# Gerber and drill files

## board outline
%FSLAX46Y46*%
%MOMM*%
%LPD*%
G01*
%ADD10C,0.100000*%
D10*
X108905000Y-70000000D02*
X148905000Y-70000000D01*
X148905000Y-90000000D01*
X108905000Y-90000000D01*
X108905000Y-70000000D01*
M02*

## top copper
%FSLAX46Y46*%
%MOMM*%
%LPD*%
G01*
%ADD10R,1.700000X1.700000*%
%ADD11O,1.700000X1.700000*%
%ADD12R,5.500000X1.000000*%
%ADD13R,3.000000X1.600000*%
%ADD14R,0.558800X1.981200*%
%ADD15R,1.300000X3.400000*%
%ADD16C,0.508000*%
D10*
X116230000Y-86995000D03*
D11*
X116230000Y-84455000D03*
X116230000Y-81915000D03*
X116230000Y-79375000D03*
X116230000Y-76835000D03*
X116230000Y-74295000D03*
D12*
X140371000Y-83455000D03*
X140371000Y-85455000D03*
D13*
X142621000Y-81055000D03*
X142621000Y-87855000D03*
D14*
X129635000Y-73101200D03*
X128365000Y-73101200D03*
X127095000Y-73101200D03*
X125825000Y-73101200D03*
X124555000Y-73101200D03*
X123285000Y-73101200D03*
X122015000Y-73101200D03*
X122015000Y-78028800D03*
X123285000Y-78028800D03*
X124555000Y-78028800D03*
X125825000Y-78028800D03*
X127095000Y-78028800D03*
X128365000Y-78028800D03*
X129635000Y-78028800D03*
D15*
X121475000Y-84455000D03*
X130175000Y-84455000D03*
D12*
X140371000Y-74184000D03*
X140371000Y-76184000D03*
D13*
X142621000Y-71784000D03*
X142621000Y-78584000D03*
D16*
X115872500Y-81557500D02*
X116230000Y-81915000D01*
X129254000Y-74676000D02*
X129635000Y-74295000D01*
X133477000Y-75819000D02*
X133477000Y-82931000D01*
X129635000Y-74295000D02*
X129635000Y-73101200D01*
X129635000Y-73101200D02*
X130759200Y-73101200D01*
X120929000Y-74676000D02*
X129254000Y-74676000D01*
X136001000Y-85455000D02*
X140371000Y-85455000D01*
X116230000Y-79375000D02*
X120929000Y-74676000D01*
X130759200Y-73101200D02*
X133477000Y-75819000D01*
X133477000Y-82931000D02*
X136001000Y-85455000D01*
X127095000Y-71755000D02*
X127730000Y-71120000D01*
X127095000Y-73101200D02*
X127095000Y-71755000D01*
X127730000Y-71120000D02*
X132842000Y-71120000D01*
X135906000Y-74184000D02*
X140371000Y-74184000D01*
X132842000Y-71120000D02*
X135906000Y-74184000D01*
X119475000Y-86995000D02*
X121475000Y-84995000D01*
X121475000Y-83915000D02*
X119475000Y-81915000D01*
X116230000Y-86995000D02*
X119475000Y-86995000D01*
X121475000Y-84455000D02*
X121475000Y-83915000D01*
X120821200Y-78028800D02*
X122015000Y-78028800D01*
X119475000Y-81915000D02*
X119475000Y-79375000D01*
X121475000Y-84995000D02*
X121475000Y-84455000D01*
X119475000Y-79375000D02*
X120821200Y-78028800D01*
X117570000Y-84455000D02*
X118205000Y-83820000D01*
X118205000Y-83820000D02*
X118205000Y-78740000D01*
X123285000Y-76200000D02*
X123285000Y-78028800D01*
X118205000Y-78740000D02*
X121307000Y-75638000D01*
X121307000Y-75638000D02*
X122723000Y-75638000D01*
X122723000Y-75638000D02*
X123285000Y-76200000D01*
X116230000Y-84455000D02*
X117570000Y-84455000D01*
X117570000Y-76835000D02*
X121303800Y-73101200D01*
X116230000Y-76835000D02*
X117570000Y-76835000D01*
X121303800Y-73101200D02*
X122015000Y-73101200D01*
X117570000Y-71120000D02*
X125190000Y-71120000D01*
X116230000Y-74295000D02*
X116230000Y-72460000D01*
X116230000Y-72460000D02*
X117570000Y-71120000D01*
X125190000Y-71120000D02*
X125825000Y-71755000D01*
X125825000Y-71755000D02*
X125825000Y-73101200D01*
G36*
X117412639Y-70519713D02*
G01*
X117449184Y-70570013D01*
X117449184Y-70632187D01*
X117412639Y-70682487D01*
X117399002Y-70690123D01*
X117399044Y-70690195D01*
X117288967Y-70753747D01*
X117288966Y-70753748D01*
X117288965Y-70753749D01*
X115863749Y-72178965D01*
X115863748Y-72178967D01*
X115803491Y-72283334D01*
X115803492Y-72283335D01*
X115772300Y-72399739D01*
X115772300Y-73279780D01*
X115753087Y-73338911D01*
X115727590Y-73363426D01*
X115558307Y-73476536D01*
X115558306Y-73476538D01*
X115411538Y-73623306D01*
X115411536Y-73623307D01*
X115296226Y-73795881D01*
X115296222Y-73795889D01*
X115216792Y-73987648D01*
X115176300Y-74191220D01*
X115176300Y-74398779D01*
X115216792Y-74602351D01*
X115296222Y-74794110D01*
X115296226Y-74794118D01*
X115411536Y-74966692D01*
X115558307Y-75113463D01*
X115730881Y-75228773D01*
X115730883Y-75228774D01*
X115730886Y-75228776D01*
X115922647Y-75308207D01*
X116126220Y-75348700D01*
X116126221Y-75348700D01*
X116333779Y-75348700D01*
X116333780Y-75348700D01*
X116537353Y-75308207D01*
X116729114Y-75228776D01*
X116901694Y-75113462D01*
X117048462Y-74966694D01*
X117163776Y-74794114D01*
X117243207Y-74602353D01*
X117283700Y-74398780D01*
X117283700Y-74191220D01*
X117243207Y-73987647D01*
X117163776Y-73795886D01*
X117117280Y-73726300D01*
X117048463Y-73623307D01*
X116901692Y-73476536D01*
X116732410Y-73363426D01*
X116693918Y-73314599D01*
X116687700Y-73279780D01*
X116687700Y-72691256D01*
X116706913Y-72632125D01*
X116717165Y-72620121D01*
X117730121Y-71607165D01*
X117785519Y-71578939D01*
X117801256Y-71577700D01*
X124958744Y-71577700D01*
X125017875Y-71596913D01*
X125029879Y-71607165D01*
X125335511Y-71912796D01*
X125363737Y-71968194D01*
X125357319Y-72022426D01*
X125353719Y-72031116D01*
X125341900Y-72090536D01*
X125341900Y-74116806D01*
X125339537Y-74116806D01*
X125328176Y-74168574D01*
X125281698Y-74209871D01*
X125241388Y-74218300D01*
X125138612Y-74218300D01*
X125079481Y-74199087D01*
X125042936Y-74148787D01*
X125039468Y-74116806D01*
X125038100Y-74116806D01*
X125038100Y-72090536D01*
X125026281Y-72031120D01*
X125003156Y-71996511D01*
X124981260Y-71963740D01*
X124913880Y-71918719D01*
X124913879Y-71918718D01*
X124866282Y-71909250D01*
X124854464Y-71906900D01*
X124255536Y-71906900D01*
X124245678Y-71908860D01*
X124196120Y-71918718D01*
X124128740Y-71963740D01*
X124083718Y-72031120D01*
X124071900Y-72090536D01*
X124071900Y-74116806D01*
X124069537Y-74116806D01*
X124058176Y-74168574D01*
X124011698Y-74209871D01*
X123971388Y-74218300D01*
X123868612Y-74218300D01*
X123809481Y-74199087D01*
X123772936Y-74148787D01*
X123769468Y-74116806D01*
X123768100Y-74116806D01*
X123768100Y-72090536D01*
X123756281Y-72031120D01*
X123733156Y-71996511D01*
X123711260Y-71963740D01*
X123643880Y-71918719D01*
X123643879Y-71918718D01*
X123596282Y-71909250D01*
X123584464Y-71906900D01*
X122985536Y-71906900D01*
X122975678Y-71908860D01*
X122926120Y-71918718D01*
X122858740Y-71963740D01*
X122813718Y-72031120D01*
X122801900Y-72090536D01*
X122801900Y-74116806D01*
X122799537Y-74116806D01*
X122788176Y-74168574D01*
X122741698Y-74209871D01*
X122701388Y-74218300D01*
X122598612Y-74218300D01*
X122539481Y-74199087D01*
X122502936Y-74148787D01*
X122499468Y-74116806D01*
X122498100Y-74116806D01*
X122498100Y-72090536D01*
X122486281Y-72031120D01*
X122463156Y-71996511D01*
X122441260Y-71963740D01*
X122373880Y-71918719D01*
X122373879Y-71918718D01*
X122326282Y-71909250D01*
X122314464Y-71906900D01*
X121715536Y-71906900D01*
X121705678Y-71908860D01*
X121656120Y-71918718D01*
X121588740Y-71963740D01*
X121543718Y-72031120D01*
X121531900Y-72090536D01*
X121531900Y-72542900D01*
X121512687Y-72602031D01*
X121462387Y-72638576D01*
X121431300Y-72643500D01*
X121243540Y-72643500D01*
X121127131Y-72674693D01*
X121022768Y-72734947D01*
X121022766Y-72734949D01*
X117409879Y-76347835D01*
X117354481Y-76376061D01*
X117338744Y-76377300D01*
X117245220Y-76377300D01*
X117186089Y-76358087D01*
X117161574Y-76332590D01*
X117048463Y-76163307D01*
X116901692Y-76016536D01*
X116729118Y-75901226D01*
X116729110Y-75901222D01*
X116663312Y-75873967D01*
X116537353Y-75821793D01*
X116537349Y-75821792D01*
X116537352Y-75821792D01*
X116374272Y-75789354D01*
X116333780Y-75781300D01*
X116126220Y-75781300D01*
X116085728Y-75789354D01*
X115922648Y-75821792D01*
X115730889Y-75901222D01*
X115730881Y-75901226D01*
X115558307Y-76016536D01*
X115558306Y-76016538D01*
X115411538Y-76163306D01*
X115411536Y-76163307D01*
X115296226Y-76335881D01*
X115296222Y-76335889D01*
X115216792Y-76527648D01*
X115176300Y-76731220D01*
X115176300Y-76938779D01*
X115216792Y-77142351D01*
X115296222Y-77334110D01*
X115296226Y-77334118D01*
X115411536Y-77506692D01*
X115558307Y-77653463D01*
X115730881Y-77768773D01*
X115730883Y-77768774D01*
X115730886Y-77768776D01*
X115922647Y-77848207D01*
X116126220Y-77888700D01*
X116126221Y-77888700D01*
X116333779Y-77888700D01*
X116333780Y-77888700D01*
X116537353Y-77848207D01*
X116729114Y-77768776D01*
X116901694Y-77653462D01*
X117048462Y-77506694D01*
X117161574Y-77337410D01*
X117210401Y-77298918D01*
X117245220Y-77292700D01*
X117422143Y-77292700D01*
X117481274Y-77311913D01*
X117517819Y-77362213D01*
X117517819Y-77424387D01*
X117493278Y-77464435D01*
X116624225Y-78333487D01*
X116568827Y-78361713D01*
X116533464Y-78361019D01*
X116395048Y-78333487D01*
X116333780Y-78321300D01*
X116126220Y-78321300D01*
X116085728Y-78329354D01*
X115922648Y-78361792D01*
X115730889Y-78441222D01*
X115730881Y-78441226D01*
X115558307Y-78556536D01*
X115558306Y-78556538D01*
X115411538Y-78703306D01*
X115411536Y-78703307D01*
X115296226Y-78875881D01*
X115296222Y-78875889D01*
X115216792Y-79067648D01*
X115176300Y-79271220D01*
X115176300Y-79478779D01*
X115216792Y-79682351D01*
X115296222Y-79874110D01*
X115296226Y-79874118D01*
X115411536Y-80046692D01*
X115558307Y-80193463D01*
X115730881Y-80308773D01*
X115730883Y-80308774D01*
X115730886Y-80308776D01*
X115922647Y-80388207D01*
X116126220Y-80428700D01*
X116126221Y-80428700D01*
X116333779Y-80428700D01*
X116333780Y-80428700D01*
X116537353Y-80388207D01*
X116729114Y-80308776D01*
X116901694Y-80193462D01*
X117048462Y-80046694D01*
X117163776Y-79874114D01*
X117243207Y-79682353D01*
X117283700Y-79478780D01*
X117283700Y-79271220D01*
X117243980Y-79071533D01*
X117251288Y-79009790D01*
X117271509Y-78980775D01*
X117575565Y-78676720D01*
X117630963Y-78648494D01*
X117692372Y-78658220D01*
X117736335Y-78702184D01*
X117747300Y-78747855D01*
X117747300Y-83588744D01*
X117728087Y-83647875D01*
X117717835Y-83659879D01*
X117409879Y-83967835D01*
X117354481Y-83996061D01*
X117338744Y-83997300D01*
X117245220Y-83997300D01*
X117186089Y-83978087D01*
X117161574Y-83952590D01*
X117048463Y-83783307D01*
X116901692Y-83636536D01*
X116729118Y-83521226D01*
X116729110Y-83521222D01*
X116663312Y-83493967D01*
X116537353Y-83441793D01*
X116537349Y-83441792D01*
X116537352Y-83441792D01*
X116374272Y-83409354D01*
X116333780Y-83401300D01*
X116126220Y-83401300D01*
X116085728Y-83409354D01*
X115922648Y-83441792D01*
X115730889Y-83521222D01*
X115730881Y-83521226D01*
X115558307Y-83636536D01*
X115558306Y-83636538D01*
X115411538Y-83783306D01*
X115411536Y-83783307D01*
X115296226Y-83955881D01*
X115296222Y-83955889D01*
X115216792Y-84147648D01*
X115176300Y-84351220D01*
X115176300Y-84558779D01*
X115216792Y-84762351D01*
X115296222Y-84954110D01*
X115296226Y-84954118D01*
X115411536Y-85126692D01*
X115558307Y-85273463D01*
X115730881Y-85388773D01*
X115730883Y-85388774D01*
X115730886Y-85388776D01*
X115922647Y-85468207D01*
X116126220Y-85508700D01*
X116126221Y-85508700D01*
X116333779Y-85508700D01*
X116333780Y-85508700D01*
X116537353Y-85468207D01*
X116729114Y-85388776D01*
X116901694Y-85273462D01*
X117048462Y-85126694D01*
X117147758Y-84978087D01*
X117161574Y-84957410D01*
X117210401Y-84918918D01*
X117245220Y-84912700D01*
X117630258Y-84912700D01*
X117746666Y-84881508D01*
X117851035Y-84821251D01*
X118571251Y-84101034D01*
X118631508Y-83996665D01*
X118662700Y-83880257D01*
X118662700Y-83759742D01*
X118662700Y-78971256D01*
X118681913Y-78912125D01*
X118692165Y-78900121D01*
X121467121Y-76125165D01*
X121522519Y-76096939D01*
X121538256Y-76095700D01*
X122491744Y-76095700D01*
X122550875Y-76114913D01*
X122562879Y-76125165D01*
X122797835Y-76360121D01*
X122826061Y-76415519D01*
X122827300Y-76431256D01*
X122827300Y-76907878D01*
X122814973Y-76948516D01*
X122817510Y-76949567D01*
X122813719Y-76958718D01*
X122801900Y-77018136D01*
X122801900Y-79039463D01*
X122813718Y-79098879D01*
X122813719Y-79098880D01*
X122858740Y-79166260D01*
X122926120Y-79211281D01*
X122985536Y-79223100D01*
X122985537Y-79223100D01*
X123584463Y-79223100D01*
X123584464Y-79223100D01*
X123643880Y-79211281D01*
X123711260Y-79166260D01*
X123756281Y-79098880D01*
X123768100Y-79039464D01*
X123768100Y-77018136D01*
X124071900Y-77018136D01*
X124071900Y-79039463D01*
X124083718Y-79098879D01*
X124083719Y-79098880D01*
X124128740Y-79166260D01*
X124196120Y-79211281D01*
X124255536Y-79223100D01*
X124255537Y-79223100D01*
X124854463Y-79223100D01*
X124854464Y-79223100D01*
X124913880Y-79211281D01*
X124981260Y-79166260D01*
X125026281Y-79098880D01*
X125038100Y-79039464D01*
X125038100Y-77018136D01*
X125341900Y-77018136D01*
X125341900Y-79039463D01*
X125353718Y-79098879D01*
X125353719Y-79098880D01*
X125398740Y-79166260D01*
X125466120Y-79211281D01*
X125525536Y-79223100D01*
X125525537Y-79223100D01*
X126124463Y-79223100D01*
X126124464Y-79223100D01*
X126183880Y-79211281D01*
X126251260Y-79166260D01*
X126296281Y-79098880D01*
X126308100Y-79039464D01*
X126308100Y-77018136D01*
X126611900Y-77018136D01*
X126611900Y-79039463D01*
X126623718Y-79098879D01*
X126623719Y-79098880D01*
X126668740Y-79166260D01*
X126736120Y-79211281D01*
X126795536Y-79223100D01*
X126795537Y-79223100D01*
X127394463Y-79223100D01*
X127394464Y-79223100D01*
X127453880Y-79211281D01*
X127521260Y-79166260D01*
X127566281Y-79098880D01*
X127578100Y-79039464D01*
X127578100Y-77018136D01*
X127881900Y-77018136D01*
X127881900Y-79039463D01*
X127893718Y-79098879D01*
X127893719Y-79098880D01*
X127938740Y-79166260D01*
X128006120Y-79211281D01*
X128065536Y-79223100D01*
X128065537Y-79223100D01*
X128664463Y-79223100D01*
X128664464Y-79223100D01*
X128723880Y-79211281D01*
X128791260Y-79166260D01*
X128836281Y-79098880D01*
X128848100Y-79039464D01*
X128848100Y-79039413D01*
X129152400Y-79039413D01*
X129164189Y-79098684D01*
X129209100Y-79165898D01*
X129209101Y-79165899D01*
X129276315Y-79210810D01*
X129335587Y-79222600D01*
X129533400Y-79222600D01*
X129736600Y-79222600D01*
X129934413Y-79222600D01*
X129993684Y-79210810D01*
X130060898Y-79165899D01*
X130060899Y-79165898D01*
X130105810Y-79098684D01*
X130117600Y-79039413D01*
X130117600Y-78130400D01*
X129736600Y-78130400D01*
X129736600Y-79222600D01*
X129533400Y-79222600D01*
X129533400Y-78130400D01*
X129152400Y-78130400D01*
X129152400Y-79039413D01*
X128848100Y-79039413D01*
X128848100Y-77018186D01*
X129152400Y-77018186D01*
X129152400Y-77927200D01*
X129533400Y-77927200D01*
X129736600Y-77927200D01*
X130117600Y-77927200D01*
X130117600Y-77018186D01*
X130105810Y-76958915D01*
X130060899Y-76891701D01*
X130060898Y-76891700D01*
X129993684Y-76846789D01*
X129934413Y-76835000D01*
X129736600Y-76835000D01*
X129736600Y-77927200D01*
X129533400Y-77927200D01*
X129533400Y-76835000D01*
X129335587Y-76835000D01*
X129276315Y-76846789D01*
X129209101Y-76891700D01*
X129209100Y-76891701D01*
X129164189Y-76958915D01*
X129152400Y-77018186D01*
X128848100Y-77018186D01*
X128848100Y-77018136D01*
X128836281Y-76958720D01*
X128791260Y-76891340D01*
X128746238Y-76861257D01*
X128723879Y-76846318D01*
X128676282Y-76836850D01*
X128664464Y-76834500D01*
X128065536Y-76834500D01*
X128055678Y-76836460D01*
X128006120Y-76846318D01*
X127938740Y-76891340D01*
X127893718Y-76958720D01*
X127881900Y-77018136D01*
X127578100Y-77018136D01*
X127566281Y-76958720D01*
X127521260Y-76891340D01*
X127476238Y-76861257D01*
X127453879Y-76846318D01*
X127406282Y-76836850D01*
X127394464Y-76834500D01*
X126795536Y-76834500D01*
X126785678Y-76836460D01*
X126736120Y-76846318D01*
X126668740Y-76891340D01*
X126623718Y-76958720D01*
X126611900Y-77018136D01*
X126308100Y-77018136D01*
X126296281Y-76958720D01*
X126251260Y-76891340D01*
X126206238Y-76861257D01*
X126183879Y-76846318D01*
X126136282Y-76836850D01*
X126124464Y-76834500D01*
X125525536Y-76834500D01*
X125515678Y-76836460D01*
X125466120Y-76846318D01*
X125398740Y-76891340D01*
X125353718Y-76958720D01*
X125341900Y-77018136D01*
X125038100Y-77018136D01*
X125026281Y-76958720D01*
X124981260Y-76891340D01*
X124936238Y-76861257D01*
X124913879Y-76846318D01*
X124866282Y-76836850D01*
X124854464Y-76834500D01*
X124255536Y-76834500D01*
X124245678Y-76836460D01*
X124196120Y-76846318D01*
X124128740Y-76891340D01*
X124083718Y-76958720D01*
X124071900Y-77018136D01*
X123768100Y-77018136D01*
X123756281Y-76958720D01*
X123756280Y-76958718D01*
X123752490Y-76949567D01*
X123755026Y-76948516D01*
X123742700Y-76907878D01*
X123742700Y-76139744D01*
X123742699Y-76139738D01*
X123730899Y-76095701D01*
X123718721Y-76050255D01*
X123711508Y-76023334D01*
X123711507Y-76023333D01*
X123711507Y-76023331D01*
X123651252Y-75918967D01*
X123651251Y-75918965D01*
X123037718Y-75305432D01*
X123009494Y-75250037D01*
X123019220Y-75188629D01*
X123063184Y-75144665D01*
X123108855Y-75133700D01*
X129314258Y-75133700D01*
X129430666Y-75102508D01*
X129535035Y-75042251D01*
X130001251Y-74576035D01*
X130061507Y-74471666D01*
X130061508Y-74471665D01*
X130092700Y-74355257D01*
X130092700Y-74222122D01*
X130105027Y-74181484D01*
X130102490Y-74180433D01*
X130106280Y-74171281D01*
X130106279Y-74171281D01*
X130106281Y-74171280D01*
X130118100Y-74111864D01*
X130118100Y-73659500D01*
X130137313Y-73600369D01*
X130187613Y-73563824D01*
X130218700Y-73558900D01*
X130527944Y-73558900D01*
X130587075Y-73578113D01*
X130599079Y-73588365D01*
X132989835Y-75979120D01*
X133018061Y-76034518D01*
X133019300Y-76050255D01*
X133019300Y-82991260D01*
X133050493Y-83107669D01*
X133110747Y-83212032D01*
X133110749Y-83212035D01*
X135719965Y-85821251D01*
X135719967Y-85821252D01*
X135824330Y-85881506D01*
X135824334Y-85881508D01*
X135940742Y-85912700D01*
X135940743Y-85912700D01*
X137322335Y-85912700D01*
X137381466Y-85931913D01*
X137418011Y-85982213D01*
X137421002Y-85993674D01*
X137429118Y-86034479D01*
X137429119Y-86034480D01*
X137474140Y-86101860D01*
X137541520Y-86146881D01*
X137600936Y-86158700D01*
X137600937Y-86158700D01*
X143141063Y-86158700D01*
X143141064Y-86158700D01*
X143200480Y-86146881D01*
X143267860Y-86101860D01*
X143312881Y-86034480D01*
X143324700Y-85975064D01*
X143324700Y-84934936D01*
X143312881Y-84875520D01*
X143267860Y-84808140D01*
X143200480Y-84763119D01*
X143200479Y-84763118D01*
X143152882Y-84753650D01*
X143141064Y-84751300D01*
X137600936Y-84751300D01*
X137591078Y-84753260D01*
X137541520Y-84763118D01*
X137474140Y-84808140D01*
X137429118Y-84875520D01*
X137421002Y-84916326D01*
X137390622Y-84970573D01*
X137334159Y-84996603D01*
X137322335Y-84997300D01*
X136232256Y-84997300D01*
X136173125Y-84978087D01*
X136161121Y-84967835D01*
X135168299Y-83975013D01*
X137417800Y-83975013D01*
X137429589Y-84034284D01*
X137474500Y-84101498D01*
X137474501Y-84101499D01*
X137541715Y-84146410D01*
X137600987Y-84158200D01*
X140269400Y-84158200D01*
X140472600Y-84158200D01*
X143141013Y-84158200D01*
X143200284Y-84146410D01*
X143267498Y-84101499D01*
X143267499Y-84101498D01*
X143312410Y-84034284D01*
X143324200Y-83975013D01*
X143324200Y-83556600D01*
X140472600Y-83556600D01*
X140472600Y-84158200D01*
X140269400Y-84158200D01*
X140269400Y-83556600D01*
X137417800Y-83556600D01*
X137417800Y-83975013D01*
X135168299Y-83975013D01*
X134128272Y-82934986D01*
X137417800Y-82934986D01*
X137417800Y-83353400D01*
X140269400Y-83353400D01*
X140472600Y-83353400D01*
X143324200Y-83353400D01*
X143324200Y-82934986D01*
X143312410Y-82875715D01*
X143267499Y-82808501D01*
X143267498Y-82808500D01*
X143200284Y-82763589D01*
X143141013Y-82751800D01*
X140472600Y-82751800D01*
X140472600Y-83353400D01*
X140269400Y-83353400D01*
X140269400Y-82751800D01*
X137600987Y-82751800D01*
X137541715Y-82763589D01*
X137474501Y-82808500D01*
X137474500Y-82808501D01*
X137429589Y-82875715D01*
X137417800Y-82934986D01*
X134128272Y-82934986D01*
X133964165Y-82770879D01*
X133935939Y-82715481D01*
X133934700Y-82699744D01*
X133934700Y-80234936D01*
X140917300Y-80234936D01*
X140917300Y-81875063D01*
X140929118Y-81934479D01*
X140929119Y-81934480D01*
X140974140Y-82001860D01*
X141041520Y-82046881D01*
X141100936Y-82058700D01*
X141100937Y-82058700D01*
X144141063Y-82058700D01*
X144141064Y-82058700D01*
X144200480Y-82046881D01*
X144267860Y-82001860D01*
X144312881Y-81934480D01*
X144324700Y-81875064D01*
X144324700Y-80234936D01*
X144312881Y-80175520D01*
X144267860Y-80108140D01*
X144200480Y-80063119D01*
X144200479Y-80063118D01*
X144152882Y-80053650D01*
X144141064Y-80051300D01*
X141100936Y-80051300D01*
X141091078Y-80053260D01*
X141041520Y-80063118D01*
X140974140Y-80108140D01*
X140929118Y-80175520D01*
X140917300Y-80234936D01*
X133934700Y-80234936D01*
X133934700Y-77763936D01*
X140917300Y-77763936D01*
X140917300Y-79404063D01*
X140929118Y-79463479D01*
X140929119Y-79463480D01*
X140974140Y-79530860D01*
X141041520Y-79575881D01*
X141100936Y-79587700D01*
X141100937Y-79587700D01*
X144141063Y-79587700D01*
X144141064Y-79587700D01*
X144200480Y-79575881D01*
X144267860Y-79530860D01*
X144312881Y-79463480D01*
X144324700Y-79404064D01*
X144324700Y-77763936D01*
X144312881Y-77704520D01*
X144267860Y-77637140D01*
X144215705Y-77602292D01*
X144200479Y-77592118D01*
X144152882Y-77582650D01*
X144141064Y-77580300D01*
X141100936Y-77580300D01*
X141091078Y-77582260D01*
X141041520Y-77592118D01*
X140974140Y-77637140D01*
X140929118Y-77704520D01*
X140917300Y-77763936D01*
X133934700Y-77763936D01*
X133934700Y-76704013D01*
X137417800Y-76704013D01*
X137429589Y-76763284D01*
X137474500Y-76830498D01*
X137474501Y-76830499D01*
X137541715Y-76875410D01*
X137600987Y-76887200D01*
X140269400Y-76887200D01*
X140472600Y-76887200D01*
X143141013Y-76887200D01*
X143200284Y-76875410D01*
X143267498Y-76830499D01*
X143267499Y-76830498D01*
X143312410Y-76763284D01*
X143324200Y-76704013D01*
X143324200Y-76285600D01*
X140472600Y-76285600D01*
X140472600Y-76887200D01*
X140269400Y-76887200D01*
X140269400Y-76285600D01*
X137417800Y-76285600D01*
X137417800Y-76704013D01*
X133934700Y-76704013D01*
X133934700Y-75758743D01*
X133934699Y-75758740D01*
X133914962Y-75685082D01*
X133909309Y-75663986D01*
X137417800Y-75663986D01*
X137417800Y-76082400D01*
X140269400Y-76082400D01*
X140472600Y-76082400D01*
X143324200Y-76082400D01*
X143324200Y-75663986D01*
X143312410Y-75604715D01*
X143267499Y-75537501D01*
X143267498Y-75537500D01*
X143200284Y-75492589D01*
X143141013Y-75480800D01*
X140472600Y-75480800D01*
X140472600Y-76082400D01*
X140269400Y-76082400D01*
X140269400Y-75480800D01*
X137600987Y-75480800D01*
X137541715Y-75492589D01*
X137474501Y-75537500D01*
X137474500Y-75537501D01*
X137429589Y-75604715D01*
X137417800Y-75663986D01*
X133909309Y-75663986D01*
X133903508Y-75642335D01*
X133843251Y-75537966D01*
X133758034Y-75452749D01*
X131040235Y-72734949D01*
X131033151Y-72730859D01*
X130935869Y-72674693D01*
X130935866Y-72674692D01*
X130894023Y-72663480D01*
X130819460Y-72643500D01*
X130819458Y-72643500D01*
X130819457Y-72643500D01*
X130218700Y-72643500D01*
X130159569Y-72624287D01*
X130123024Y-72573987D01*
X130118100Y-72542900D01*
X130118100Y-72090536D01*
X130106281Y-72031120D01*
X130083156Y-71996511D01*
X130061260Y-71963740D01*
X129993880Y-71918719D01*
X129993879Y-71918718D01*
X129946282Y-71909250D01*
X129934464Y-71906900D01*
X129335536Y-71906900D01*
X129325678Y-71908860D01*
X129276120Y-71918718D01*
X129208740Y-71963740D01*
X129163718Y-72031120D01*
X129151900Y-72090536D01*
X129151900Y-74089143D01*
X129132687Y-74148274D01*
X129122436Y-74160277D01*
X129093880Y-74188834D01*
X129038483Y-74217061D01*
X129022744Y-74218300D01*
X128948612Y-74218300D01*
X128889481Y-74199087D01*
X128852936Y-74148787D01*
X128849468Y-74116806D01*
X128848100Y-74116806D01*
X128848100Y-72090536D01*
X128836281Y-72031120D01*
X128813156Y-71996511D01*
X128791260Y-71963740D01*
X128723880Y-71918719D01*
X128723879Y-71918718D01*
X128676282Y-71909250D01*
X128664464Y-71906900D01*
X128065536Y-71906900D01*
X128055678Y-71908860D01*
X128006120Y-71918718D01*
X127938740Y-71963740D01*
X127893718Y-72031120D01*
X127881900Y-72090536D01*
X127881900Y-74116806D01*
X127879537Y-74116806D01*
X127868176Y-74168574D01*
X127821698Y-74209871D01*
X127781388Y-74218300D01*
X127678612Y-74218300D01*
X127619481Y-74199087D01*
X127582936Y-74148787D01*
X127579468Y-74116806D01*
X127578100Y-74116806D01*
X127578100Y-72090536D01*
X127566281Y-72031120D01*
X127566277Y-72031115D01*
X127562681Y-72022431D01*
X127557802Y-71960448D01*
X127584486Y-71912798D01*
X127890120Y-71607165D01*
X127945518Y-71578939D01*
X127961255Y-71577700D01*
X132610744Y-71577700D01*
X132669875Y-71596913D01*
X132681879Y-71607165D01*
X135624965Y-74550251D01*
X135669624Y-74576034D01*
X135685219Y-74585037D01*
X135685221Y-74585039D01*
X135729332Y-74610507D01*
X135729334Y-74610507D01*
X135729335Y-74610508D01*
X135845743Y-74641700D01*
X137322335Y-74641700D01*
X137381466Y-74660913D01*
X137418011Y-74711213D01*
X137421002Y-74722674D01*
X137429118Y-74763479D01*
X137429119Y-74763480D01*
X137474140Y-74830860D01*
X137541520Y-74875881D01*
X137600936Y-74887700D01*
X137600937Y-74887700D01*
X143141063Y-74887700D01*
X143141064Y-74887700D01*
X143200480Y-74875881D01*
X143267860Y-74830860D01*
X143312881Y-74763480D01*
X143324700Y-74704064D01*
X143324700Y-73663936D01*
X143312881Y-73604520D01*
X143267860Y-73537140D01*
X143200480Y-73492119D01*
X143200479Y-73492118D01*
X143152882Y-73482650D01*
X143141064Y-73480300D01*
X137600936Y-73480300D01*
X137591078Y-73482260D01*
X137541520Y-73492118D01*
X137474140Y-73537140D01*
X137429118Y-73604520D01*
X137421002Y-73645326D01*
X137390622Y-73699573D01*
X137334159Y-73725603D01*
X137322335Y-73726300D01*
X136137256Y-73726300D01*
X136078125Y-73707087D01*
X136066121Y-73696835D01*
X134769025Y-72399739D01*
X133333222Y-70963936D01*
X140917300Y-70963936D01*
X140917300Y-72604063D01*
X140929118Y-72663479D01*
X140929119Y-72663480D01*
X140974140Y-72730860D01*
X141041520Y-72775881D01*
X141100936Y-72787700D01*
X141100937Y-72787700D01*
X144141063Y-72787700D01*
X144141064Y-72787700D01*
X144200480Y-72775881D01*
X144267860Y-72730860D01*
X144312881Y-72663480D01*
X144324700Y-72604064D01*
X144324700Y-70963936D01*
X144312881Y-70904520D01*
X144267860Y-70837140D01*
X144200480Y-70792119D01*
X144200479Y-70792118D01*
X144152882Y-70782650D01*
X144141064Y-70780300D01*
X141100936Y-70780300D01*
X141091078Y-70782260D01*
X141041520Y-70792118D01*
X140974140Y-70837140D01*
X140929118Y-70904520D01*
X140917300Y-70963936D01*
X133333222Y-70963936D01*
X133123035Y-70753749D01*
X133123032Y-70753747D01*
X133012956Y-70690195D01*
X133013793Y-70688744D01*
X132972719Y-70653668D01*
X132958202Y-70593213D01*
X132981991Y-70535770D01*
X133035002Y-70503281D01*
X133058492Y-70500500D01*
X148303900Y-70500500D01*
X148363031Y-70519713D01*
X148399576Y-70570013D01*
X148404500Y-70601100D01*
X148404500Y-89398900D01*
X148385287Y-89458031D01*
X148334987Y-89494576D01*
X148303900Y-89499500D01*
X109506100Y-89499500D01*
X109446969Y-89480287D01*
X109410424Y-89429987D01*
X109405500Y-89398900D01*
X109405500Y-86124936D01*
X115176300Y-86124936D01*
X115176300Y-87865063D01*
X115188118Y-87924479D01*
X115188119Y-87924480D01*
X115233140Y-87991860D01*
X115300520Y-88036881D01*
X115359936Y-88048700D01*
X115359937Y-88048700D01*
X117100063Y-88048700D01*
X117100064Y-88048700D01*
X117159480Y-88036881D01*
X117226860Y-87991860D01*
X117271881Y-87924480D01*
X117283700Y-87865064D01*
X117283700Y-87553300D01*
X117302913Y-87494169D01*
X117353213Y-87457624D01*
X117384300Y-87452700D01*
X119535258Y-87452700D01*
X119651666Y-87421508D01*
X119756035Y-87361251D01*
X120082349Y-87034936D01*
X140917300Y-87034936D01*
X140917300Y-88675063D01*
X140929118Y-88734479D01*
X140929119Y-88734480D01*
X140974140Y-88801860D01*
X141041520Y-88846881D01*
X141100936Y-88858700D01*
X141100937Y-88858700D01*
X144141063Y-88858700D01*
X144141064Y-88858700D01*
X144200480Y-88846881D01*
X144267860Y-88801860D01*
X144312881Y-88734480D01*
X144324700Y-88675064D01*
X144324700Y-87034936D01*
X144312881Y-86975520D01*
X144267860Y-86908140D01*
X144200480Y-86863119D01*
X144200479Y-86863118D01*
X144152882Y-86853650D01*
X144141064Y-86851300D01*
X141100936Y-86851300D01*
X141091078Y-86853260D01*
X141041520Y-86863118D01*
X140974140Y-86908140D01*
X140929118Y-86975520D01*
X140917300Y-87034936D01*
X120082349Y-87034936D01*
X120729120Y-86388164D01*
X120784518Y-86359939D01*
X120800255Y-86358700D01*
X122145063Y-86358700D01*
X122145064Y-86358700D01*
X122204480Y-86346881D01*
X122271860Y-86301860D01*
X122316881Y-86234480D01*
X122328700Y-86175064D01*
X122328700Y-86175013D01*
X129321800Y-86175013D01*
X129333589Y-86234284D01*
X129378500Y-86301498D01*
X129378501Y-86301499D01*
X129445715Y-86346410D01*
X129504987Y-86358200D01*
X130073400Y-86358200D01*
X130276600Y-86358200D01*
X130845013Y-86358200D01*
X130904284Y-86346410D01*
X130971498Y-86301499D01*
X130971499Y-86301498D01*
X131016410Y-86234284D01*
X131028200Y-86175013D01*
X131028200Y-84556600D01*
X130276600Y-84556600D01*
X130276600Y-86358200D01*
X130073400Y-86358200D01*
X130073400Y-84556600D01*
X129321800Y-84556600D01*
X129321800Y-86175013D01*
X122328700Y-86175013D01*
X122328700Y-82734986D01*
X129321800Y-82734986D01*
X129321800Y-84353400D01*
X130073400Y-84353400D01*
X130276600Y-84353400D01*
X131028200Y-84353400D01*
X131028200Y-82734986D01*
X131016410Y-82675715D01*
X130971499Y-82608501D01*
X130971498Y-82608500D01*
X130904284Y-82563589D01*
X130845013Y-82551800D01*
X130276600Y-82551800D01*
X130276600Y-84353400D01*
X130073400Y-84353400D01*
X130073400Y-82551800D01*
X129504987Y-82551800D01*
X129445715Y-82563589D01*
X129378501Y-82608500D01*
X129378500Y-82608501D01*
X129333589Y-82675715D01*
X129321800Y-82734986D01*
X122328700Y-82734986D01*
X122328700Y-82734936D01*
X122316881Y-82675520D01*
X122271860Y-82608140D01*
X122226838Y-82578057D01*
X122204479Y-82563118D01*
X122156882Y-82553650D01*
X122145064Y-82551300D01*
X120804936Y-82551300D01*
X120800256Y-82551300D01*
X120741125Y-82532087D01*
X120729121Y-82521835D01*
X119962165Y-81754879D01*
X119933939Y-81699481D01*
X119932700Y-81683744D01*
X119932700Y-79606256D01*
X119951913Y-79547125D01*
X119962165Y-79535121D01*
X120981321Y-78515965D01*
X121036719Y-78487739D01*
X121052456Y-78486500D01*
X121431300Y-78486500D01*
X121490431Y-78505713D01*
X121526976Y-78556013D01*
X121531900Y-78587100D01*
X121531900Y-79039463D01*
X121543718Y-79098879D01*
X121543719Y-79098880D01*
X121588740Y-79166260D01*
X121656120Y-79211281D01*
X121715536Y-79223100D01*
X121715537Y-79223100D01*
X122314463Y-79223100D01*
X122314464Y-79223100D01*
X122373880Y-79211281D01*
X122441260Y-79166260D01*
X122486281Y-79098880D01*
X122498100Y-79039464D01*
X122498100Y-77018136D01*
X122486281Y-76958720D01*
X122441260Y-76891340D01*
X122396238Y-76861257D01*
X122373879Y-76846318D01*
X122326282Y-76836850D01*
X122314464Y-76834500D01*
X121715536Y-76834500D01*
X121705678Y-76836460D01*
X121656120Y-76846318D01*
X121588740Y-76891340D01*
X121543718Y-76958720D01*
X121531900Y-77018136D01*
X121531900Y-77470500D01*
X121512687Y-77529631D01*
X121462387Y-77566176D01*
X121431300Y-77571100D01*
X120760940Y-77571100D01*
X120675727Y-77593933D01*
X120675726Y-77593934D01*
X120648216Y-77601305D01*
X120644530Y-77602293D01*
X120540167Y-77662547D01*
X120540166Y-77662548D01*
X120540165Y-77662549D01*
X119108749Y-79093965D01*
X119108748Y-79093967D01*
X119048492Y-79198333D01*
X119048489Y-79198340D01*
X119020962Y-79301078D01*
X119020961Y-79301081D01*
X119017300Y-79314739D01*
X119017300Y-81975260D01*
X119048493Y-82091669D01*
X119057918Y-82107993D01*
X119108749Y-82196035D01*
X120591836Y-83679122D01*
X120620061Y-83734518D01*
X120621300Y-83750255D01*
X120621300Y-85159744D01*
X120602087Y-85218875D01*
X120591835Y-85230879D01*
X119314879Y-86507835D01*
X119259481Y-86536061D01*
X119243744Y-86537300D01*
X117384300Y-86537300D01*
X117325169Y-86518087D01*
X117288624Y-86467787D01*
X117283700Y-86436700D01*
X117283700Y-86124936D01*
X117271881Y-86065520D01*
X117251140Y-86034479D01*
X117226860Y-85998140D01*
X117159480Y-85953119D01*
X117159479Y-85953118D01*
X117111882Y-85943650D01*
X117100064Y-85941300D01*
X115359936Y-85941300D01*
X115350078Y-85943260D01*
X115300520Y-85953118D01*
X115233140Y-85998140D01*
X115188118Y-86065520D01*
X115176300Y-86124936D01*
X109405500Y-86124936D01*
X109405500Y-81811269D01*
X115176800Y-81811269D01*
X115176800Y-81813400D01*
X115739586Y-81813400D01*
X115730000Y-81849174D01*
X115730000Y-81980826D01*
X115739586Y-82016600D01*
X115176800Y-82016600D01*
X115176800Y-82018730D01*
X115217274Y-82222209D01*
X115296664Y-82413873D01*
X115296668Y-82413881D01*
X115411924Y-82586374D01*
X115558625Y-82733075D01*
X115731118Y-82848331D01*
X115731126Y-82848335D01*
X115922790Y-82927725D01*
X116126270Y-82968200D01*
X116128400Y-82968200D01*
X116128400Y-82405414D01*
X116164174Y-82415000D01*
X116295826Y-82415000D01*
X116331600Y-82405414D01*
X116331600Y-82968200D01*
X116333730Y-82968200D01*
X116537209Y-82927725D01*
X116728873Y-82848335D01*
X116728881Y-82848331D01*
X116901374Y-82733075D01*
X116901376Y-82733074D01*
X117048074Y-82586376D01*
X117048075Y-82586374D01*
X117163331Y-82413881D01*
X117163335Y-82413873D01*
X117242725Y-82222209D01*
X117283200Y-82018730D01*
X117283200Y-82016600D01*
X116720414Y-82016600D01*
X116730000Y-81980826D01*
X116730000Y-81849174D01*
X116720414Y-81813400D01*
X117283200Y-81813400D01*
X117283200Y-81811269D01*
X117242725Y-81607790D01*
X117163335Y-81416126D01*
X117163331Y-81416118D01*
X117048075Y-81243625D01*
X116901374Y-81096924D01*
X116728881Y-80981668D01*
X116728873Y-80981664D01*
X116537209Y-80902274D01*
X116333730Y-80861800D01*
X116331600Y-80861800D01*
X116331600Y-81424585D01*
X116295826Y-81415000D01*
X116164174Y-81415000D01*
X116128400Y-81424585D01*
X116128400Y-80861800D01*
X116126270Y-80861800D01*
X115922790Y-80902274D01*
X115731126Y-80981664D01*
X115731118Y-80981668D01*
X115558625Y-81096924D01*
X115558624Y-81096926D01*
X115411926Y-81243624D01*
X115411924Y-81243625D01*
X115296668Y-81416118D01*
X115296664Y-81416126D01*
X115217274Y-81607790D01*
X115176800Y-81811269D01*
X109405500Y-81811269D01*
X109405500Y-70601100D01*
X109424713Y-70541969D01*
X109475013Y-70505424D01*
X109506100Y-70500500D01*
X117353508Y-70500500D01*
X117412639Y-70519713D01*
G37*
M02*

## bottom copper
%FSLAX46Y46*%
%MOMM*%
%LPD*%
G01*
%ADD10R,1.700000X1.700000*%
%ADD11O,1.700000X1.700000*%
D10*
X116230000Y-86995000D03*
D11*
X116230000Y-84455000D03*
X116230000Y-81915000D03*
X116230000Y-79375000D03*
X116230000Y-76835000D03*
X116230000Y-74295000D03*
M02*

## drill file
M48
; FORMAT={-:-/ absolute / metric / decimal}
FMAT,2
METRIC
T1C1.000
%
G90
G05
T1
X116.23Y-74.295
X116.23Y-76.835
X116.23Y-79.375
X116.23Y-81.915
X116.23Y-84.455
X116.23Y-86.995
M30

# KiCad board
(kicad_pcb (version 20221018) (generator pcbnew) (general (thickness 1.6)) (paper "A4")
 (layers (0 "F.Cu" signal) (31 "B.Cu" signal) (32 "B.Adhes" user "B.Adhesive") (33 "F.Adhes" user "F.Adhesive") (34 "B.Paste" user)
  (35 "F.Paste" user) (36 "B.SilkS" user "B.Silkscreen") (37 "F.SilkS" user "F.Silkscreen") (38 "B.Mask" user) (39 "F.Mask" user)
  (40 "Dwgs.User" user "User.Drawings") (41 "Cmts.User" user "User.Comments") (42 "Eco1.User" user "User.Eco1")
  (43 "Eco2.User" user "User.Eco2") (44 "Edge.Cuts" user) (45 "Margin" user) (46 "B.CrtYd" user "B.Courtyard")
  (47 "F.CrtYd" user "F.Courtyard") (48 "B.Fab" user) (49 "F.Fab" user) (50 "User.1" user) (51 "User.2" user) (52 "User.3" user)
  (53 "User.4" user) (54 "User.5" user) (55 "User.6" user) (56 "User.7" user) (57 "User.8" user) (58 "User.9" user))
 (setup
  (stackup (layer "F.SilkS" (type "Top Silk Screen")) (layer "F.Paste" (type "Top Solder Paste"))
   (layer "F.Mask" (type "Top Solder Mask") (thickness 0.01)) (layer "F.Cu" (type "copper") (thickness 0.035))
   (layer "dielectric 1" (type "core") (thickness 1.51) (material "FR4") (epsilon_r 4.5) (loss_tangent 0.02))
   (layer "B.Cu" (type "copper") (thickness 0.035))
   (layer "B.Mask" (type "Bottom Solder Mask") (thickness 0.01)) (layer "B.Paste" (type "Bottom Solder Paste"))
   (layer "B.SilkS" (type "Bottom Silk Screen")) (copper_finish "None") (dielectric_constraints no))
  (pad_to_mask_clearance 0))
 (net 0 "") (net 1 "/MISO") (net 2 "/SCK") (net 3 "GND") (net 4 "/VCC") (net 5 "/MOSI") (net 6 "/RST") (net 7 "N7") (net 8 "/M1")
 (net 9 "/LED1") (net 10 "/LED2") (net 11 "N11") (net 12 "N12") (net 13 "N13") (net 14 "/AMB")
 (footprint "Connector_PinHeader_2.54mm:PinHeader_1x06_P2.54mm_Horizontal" (layer "F.Cu") (at 116.23 86.995 180)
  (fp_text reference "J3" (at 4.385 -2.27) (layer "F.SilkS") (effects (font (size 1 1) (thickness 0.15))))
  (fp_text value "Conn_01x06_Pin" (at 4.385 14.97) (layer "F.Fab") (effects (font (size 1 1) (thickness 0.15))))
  (pad "1" thru_hole rect (at 0 0 180) (size 1.7 1.7) (drill 1) (layers "*.Cu" "*.Mask") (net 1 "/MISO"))
  (pad "2" thru_hole oval (at 0 2.54 180) (size 1.7 1.7) (drill 1) (layers "*.Cu" "*.Mask") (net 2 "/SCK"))
  (pad "3" thru_hole oval (at 0 5.08 180) (size 1.7 1.7) (drill 1) (layers "*.Cu" "*.Mask") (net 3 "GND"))
  (pad "4" thru_hole oval (at 0 7.62 180) (size 1.7 1.7) (drill 1) (layers "*.Cu" "*.Mask") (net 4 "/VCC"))
  (pad "5" thru_hole oval (at 0 10.16 180) (size 1.7 1.7) (drill 1) (layers "*.Cu" "*.Mask") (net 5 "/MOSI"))
  (pad "6" thru_hole oval (at 0 12.7 180) (size 1.7 1.7) (drill 1) (layers "*.Cu" "*.Mask") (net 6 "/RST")))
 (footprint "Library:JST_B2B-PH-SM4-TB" (layer "F.Cu") (at 142.621 84.455 -90)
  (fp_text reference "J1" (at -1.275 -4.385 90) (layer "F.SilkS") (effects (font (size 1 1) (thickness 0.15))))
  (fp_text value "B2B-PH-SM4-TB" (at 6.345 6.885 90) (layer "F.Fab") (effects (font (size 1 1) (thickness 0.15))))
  (pad "1" smd rect (at -1 2.25 270) (size 1 5.5) (layers "F.Cu" "F.Paste" "F.Mask") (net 3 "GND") (solder_mask_margin 0.102))
  (pad "2" smd rect (at 1 2.25 270) (size 1 5.5) (layers "F.Cu" "F.Paste" "F.Mask") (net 4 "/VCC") (solder_mask_margin 0.102))
  (pad "S1" smd rect (at -3.4 0 270) (size 1.6 3) (layers "F.Cu" "F.Paste" "F.Mask") (solder_mask_margin 0.102))
  (pad "S2" smd rect (at 3.4 0 270) (size 1.6 3) (layers "F.Cu" "F.Paste" "F.Mask") (solder_mask_margin 0.102)))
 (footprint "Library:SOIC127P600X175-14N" (layer "F.Cu") (at 125.825 75.565 -90)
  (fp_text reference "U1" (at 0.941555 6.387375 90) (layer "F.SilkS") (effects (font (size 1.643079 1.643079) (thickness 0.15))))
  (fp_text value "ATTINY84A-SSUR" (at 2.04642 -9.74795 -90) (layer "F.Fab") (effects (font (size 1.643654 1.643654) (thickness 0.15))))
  (pad "1" smd rect (at -2.4638 -3.81 270) (size 1.9812 0.5588) (layers "F.Cu" "F.Paste" "F.Mask") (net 4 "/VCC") (solder_mask_margin 0.102))
  (pad "2" smd rect (at -2.4638 -2.54 270) (size 1.9812 0.5588) (layers "F.Cu" "F.Paste" "F.Mask") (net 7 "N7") (solder_mask_margin 0.102))
  (pad "3" smd rect (at -2.4638 -1.27 270) (size 1.9812 0.5588) (layers "F.Cu" "F.Paste" "F.Mask") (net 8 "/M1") (solder_mask_margin 0.102))
  (pad "4" smd rect (at -2.4638 0 270) (size 1.9812 0.5588) (layers "F.Cu" "F.Paste" "F.Mask") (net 6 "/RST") (solder_mask_margin 0.102))
  (pad "5" smd rect (at -2.4638 1.27 270) (size 1.9812 0.5588) (layers "F.Cu" "F.Paste" "F.Mask") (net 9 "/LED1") (solder_mask_margin 0.102))
  (pad "6" smd rect (at -2.4638 2.54 270) (size 1.9812 0.5588) (layers "F.Cu" "F.Paste" "F.Mask") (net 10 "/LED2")
   (solder_mask_margin 0.102))
  (pad "7" smd rect (at -2.4638 3.81 270) (size 1.9812 0.5588) (layers "F.Cu" "F.Paste" "F.Mask") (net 5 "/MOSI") (solder_mask_margin 0.102))
  (pad "8" smd rect (at 2.4638 3.81 270) (size 1.9812 0.5588) (layers "F.Cu" "F.Paste" "F.Mask") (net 1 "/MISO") (solder_mask_margin 0.102))
  (pad "9" smd rect (at 2.4638 2.54 270) (size 1.9812 0.5588) (layers "F.Cu" "F.Paste" "F.Mask") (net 2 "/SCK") (solder_mask_margin 0.102))
  (pad "10" smd rect (at 2.4638 1.27 270) (size 1.9812 0.5588) (layers "F.Cu" "F.Paste" "F.Mask") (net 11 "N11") (solder_mask_margin 0.102))
  (pad "11" smd rect (at 2.4638 0 270) (size 1.9812 0.5588) (layers "F.Cu" "F.Paste" "F.Mask") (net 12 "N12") (solder_mask_margin 0.102))
  (pad "12" smd rect (at 2.4638 -1.27 270) (size 1.9812 0.5588) (layers "F.Cu" "F.Paste" "F.Mask") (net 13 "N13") (solder_mask_margin 0.102))
  (pad "13" smd rect (at 2.4638 -2.54 270) (size 1.9812 0.5588) (layers "F.Cu" "F.Paste" "F.Mask") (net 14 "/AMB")
   (solder_mask_margin 0.102))
  (pad "14" smd rect (at 2.4638 -3.81 270) (size 1.9812 0.5588) (layers "F.Cu" "F.Paste" "F.Mask") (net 3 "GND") (solder_mask_margin 0.102)))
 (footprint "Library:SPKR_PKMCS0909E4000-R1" (layer "F.Cu") (at 125.825 84.455)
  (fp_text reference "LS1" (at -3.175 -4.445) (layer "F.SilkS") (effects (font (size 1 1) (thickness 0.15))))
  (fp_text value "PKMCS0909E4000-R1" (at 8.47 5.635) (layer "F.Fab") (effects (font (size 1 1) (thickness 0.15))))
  (pad "1" smd rect (at -4.35 0) (size 1.3 3.4) (layers "F.Cu" "F.Paste" "F.Mask") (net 1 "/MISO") (solder_mask_margin 0.102))
  (pad "2" smd rect (at 4.35 0) (size 1.3 3.4) (layers "F.Cu" "F.Paste" "F.Mask") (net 3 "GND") (solder_mask_margin 0.102)))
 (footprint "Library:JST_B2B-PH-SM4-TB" (layer "F.Cu") (at 142.621 75.184 -90)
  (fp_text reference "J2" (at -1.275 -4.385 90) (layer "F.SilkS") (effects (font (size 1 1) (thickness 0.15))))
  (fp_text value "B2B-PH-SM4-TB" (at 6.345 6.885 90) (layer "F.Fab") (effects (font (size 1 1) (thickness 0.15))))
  (pad "1" smd rect (at -1 2.25 270) (size 1 5.5) (layers "F.Cu" "F.Paste" "F.Mask") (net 8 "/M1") (solder_mask_margin 0.102))
  (pad "2" smd rect (at 1 2.25 270) (size 1 5.5) (layers "F.Cu" "F.Paste" "F.Mask") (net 3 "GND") (solder_mask_margin 0.102))
  (pad "S1" smd rect (at -3.4 0 270) (size 1.6 3) (layers "F.Cu" "F.Paste" "F.Mask") (solder_mask_margin 0.102))
  (pad "S2" smd rect (at 3.4 0 270) (size 1.6 3) (layers "F.Cu" "F.Paste" "F.Mask") (solder_mask_margin 0.102)))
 (gr_rect (start 108.905 70) (end 148.905 90) (stroke (width 0.1) (type default)) (fill none) (layer "Edge.Cuts"))
 (segment (start 115.8725 81.5575) (end 116.23 81.915) (width 0.508) (layer "F.Cu") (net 3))
 (segment (start 129.254 74.676) (end 129.635 74.295) (width 0.508) (layer "F.Cu") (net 4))
 (segment (start 133.477 75.819) (end 133.477 82.931) (width 0.508) (layer "F.Cu") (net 4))
 (segment (start 129.635 74.295) (end 129.635 73.1012) (width 0.508) (layer "F.Cu") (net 4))
 (segment (start 129.635 73.1012) (end 130.7592 73.1012) (width 0.508) (layer "F.Cu") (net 4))
 (segment (start 120.929 74.676) (end 129.254 74.676) (width 0.508) (layer "F.Cu") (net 4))
 (segment (start 136.001 85.455) (end 140.371 85.455) (width 0.508) (layer "F.Cu") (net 4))
 (segment (start 116.23 79.375) (end 120.929 74.676) (width 0.508) (layer "F.Cu") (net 4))
 (segment (start 130.7592 73.1012) (end 133.477 75.819) (width 0.508) (layer "F.Cu") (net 4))
 (segment (start 133.477 82.931) (end 136.001 85.455) (width 0.508) (layer "F.Cu") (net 4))
 (segment (start 127.095 71.755) (end 127.73 71.12) (width 0.508) (layer "F.Cu") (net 8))
 (segment (start 127.095 73.1012) (end 127.095 71.755) (width 0.508) (layer "F.Cu") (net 8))
 (segment (start 127.73 71.12) (end 132.842 71.12) (width 0.508) (layer "F.Cu") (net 8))
 (segment (start 135.906 74.184) (end 140.371 74.184) (width 0.508) (layer "F.Cu") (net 8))
 (segment (start 132.842 71.12) (end 135.906 74.184) (width 0.508) (layer "F.Cu") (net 8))
 (segment (start 119.475 86.995) (end 121.475 84.995) (width 0.508) (layer "F.Cu") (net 1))
 (segment (start 121.475 83.915) (end 119.475 81.915) (width 0.508) (layer "F.Cu") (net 1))
 (segment (start 116.23 86.995) (end 119.475 86.995) (width 0.508) (layer "F.Cu") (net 1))
 (segment (start 121.475 84.455) (end 121.475 83.915) (width 0.508) (layer "F.Cu") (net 1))
 (segment (start 120.8212 78.0288) (end 122.015 78.0288) (width 0.508) (layer "F.Cu") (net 1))
 (segment (start 119.475 81.915) (end 119.475 79.375) (width 0.508) (layer "F.Cu") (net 1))
 (segment (start 121.475 84.995) (end 121.475 84.455) (width 0.508) (layer "F.Cu") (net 1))
 (segment (start 119.475 79.375) (end 120.8212 78.0288) (width 0.508) (layer "F.Cu") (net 1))
 (segment (start 117.57 84.455) (end 118.205 83.82) (width 0.508) (layer "F.Cu") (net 2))
 (segment (start 118.205 83.82) (end 118.205 78.74) (width 0.508) (layer "F.Cu") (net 2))
 (segment (start 123.285 76.2) (end 123.285 78.0288) (width 0.508) (layer "F.Cu") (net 2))
 (segment (start 118.205 78.74) (end 121.307 75.638) (width 0.508) (layer "F.Cu") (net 2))
 (segment (start 121.307 75.638) (end 122.723 75.638) (width 0.508) (layer "F.Cu") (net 2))
 (segment (start 122.723 75.638) (end 123.285 76.2) (width 0.508) (layer "F.Cu") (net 2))
 (segment (start 116.23 84.455) (end 117.57 84.455) (width 0.508) (layer "F.Cu") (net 2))
 (segment (start 117.57 76.835) (end 121.3038 73.1012) (width 0.508) (layer "F.Cu") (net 5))
 (segment (start 116.23 76.835) (end 117.57 76.835) (width 0.508) (layer "F.Cu") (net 5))
 (segment (start 121.3038 73.1012) (end 122.015 73.1012) (width 0.508) (layer "F.Cu") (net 5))
 (segment (start 117.57 71.12) (end 125.19 71.12) (width 0.508) (layer "F.Cu") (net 6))
 (segment (start 116.23 74.295) (end 116.23 72.46) (width 0.508) (layer "F.Cu") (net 6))
 (segment (start 116.23 72.46) (end 117.57 71.12) (width 0.508) (layer "F.Cu") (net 6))
 (segment (start 125.19 71.12) (end 125.825 71.755) (width 0.508) (layer "F.Cu") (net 6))
 (segment (start 125.825 71.755) (end 125.825 73.1012) (width 0.508) (layer "F.Cu") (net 6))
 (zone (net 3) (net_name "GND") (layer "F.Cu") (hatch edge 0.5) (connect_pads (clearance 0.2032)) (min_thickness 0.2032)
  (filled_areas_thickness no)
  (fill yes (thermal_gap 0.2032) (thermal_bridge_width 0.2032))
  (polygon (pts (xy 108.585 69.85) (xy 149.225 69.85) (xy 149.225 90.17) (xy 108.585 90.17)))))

